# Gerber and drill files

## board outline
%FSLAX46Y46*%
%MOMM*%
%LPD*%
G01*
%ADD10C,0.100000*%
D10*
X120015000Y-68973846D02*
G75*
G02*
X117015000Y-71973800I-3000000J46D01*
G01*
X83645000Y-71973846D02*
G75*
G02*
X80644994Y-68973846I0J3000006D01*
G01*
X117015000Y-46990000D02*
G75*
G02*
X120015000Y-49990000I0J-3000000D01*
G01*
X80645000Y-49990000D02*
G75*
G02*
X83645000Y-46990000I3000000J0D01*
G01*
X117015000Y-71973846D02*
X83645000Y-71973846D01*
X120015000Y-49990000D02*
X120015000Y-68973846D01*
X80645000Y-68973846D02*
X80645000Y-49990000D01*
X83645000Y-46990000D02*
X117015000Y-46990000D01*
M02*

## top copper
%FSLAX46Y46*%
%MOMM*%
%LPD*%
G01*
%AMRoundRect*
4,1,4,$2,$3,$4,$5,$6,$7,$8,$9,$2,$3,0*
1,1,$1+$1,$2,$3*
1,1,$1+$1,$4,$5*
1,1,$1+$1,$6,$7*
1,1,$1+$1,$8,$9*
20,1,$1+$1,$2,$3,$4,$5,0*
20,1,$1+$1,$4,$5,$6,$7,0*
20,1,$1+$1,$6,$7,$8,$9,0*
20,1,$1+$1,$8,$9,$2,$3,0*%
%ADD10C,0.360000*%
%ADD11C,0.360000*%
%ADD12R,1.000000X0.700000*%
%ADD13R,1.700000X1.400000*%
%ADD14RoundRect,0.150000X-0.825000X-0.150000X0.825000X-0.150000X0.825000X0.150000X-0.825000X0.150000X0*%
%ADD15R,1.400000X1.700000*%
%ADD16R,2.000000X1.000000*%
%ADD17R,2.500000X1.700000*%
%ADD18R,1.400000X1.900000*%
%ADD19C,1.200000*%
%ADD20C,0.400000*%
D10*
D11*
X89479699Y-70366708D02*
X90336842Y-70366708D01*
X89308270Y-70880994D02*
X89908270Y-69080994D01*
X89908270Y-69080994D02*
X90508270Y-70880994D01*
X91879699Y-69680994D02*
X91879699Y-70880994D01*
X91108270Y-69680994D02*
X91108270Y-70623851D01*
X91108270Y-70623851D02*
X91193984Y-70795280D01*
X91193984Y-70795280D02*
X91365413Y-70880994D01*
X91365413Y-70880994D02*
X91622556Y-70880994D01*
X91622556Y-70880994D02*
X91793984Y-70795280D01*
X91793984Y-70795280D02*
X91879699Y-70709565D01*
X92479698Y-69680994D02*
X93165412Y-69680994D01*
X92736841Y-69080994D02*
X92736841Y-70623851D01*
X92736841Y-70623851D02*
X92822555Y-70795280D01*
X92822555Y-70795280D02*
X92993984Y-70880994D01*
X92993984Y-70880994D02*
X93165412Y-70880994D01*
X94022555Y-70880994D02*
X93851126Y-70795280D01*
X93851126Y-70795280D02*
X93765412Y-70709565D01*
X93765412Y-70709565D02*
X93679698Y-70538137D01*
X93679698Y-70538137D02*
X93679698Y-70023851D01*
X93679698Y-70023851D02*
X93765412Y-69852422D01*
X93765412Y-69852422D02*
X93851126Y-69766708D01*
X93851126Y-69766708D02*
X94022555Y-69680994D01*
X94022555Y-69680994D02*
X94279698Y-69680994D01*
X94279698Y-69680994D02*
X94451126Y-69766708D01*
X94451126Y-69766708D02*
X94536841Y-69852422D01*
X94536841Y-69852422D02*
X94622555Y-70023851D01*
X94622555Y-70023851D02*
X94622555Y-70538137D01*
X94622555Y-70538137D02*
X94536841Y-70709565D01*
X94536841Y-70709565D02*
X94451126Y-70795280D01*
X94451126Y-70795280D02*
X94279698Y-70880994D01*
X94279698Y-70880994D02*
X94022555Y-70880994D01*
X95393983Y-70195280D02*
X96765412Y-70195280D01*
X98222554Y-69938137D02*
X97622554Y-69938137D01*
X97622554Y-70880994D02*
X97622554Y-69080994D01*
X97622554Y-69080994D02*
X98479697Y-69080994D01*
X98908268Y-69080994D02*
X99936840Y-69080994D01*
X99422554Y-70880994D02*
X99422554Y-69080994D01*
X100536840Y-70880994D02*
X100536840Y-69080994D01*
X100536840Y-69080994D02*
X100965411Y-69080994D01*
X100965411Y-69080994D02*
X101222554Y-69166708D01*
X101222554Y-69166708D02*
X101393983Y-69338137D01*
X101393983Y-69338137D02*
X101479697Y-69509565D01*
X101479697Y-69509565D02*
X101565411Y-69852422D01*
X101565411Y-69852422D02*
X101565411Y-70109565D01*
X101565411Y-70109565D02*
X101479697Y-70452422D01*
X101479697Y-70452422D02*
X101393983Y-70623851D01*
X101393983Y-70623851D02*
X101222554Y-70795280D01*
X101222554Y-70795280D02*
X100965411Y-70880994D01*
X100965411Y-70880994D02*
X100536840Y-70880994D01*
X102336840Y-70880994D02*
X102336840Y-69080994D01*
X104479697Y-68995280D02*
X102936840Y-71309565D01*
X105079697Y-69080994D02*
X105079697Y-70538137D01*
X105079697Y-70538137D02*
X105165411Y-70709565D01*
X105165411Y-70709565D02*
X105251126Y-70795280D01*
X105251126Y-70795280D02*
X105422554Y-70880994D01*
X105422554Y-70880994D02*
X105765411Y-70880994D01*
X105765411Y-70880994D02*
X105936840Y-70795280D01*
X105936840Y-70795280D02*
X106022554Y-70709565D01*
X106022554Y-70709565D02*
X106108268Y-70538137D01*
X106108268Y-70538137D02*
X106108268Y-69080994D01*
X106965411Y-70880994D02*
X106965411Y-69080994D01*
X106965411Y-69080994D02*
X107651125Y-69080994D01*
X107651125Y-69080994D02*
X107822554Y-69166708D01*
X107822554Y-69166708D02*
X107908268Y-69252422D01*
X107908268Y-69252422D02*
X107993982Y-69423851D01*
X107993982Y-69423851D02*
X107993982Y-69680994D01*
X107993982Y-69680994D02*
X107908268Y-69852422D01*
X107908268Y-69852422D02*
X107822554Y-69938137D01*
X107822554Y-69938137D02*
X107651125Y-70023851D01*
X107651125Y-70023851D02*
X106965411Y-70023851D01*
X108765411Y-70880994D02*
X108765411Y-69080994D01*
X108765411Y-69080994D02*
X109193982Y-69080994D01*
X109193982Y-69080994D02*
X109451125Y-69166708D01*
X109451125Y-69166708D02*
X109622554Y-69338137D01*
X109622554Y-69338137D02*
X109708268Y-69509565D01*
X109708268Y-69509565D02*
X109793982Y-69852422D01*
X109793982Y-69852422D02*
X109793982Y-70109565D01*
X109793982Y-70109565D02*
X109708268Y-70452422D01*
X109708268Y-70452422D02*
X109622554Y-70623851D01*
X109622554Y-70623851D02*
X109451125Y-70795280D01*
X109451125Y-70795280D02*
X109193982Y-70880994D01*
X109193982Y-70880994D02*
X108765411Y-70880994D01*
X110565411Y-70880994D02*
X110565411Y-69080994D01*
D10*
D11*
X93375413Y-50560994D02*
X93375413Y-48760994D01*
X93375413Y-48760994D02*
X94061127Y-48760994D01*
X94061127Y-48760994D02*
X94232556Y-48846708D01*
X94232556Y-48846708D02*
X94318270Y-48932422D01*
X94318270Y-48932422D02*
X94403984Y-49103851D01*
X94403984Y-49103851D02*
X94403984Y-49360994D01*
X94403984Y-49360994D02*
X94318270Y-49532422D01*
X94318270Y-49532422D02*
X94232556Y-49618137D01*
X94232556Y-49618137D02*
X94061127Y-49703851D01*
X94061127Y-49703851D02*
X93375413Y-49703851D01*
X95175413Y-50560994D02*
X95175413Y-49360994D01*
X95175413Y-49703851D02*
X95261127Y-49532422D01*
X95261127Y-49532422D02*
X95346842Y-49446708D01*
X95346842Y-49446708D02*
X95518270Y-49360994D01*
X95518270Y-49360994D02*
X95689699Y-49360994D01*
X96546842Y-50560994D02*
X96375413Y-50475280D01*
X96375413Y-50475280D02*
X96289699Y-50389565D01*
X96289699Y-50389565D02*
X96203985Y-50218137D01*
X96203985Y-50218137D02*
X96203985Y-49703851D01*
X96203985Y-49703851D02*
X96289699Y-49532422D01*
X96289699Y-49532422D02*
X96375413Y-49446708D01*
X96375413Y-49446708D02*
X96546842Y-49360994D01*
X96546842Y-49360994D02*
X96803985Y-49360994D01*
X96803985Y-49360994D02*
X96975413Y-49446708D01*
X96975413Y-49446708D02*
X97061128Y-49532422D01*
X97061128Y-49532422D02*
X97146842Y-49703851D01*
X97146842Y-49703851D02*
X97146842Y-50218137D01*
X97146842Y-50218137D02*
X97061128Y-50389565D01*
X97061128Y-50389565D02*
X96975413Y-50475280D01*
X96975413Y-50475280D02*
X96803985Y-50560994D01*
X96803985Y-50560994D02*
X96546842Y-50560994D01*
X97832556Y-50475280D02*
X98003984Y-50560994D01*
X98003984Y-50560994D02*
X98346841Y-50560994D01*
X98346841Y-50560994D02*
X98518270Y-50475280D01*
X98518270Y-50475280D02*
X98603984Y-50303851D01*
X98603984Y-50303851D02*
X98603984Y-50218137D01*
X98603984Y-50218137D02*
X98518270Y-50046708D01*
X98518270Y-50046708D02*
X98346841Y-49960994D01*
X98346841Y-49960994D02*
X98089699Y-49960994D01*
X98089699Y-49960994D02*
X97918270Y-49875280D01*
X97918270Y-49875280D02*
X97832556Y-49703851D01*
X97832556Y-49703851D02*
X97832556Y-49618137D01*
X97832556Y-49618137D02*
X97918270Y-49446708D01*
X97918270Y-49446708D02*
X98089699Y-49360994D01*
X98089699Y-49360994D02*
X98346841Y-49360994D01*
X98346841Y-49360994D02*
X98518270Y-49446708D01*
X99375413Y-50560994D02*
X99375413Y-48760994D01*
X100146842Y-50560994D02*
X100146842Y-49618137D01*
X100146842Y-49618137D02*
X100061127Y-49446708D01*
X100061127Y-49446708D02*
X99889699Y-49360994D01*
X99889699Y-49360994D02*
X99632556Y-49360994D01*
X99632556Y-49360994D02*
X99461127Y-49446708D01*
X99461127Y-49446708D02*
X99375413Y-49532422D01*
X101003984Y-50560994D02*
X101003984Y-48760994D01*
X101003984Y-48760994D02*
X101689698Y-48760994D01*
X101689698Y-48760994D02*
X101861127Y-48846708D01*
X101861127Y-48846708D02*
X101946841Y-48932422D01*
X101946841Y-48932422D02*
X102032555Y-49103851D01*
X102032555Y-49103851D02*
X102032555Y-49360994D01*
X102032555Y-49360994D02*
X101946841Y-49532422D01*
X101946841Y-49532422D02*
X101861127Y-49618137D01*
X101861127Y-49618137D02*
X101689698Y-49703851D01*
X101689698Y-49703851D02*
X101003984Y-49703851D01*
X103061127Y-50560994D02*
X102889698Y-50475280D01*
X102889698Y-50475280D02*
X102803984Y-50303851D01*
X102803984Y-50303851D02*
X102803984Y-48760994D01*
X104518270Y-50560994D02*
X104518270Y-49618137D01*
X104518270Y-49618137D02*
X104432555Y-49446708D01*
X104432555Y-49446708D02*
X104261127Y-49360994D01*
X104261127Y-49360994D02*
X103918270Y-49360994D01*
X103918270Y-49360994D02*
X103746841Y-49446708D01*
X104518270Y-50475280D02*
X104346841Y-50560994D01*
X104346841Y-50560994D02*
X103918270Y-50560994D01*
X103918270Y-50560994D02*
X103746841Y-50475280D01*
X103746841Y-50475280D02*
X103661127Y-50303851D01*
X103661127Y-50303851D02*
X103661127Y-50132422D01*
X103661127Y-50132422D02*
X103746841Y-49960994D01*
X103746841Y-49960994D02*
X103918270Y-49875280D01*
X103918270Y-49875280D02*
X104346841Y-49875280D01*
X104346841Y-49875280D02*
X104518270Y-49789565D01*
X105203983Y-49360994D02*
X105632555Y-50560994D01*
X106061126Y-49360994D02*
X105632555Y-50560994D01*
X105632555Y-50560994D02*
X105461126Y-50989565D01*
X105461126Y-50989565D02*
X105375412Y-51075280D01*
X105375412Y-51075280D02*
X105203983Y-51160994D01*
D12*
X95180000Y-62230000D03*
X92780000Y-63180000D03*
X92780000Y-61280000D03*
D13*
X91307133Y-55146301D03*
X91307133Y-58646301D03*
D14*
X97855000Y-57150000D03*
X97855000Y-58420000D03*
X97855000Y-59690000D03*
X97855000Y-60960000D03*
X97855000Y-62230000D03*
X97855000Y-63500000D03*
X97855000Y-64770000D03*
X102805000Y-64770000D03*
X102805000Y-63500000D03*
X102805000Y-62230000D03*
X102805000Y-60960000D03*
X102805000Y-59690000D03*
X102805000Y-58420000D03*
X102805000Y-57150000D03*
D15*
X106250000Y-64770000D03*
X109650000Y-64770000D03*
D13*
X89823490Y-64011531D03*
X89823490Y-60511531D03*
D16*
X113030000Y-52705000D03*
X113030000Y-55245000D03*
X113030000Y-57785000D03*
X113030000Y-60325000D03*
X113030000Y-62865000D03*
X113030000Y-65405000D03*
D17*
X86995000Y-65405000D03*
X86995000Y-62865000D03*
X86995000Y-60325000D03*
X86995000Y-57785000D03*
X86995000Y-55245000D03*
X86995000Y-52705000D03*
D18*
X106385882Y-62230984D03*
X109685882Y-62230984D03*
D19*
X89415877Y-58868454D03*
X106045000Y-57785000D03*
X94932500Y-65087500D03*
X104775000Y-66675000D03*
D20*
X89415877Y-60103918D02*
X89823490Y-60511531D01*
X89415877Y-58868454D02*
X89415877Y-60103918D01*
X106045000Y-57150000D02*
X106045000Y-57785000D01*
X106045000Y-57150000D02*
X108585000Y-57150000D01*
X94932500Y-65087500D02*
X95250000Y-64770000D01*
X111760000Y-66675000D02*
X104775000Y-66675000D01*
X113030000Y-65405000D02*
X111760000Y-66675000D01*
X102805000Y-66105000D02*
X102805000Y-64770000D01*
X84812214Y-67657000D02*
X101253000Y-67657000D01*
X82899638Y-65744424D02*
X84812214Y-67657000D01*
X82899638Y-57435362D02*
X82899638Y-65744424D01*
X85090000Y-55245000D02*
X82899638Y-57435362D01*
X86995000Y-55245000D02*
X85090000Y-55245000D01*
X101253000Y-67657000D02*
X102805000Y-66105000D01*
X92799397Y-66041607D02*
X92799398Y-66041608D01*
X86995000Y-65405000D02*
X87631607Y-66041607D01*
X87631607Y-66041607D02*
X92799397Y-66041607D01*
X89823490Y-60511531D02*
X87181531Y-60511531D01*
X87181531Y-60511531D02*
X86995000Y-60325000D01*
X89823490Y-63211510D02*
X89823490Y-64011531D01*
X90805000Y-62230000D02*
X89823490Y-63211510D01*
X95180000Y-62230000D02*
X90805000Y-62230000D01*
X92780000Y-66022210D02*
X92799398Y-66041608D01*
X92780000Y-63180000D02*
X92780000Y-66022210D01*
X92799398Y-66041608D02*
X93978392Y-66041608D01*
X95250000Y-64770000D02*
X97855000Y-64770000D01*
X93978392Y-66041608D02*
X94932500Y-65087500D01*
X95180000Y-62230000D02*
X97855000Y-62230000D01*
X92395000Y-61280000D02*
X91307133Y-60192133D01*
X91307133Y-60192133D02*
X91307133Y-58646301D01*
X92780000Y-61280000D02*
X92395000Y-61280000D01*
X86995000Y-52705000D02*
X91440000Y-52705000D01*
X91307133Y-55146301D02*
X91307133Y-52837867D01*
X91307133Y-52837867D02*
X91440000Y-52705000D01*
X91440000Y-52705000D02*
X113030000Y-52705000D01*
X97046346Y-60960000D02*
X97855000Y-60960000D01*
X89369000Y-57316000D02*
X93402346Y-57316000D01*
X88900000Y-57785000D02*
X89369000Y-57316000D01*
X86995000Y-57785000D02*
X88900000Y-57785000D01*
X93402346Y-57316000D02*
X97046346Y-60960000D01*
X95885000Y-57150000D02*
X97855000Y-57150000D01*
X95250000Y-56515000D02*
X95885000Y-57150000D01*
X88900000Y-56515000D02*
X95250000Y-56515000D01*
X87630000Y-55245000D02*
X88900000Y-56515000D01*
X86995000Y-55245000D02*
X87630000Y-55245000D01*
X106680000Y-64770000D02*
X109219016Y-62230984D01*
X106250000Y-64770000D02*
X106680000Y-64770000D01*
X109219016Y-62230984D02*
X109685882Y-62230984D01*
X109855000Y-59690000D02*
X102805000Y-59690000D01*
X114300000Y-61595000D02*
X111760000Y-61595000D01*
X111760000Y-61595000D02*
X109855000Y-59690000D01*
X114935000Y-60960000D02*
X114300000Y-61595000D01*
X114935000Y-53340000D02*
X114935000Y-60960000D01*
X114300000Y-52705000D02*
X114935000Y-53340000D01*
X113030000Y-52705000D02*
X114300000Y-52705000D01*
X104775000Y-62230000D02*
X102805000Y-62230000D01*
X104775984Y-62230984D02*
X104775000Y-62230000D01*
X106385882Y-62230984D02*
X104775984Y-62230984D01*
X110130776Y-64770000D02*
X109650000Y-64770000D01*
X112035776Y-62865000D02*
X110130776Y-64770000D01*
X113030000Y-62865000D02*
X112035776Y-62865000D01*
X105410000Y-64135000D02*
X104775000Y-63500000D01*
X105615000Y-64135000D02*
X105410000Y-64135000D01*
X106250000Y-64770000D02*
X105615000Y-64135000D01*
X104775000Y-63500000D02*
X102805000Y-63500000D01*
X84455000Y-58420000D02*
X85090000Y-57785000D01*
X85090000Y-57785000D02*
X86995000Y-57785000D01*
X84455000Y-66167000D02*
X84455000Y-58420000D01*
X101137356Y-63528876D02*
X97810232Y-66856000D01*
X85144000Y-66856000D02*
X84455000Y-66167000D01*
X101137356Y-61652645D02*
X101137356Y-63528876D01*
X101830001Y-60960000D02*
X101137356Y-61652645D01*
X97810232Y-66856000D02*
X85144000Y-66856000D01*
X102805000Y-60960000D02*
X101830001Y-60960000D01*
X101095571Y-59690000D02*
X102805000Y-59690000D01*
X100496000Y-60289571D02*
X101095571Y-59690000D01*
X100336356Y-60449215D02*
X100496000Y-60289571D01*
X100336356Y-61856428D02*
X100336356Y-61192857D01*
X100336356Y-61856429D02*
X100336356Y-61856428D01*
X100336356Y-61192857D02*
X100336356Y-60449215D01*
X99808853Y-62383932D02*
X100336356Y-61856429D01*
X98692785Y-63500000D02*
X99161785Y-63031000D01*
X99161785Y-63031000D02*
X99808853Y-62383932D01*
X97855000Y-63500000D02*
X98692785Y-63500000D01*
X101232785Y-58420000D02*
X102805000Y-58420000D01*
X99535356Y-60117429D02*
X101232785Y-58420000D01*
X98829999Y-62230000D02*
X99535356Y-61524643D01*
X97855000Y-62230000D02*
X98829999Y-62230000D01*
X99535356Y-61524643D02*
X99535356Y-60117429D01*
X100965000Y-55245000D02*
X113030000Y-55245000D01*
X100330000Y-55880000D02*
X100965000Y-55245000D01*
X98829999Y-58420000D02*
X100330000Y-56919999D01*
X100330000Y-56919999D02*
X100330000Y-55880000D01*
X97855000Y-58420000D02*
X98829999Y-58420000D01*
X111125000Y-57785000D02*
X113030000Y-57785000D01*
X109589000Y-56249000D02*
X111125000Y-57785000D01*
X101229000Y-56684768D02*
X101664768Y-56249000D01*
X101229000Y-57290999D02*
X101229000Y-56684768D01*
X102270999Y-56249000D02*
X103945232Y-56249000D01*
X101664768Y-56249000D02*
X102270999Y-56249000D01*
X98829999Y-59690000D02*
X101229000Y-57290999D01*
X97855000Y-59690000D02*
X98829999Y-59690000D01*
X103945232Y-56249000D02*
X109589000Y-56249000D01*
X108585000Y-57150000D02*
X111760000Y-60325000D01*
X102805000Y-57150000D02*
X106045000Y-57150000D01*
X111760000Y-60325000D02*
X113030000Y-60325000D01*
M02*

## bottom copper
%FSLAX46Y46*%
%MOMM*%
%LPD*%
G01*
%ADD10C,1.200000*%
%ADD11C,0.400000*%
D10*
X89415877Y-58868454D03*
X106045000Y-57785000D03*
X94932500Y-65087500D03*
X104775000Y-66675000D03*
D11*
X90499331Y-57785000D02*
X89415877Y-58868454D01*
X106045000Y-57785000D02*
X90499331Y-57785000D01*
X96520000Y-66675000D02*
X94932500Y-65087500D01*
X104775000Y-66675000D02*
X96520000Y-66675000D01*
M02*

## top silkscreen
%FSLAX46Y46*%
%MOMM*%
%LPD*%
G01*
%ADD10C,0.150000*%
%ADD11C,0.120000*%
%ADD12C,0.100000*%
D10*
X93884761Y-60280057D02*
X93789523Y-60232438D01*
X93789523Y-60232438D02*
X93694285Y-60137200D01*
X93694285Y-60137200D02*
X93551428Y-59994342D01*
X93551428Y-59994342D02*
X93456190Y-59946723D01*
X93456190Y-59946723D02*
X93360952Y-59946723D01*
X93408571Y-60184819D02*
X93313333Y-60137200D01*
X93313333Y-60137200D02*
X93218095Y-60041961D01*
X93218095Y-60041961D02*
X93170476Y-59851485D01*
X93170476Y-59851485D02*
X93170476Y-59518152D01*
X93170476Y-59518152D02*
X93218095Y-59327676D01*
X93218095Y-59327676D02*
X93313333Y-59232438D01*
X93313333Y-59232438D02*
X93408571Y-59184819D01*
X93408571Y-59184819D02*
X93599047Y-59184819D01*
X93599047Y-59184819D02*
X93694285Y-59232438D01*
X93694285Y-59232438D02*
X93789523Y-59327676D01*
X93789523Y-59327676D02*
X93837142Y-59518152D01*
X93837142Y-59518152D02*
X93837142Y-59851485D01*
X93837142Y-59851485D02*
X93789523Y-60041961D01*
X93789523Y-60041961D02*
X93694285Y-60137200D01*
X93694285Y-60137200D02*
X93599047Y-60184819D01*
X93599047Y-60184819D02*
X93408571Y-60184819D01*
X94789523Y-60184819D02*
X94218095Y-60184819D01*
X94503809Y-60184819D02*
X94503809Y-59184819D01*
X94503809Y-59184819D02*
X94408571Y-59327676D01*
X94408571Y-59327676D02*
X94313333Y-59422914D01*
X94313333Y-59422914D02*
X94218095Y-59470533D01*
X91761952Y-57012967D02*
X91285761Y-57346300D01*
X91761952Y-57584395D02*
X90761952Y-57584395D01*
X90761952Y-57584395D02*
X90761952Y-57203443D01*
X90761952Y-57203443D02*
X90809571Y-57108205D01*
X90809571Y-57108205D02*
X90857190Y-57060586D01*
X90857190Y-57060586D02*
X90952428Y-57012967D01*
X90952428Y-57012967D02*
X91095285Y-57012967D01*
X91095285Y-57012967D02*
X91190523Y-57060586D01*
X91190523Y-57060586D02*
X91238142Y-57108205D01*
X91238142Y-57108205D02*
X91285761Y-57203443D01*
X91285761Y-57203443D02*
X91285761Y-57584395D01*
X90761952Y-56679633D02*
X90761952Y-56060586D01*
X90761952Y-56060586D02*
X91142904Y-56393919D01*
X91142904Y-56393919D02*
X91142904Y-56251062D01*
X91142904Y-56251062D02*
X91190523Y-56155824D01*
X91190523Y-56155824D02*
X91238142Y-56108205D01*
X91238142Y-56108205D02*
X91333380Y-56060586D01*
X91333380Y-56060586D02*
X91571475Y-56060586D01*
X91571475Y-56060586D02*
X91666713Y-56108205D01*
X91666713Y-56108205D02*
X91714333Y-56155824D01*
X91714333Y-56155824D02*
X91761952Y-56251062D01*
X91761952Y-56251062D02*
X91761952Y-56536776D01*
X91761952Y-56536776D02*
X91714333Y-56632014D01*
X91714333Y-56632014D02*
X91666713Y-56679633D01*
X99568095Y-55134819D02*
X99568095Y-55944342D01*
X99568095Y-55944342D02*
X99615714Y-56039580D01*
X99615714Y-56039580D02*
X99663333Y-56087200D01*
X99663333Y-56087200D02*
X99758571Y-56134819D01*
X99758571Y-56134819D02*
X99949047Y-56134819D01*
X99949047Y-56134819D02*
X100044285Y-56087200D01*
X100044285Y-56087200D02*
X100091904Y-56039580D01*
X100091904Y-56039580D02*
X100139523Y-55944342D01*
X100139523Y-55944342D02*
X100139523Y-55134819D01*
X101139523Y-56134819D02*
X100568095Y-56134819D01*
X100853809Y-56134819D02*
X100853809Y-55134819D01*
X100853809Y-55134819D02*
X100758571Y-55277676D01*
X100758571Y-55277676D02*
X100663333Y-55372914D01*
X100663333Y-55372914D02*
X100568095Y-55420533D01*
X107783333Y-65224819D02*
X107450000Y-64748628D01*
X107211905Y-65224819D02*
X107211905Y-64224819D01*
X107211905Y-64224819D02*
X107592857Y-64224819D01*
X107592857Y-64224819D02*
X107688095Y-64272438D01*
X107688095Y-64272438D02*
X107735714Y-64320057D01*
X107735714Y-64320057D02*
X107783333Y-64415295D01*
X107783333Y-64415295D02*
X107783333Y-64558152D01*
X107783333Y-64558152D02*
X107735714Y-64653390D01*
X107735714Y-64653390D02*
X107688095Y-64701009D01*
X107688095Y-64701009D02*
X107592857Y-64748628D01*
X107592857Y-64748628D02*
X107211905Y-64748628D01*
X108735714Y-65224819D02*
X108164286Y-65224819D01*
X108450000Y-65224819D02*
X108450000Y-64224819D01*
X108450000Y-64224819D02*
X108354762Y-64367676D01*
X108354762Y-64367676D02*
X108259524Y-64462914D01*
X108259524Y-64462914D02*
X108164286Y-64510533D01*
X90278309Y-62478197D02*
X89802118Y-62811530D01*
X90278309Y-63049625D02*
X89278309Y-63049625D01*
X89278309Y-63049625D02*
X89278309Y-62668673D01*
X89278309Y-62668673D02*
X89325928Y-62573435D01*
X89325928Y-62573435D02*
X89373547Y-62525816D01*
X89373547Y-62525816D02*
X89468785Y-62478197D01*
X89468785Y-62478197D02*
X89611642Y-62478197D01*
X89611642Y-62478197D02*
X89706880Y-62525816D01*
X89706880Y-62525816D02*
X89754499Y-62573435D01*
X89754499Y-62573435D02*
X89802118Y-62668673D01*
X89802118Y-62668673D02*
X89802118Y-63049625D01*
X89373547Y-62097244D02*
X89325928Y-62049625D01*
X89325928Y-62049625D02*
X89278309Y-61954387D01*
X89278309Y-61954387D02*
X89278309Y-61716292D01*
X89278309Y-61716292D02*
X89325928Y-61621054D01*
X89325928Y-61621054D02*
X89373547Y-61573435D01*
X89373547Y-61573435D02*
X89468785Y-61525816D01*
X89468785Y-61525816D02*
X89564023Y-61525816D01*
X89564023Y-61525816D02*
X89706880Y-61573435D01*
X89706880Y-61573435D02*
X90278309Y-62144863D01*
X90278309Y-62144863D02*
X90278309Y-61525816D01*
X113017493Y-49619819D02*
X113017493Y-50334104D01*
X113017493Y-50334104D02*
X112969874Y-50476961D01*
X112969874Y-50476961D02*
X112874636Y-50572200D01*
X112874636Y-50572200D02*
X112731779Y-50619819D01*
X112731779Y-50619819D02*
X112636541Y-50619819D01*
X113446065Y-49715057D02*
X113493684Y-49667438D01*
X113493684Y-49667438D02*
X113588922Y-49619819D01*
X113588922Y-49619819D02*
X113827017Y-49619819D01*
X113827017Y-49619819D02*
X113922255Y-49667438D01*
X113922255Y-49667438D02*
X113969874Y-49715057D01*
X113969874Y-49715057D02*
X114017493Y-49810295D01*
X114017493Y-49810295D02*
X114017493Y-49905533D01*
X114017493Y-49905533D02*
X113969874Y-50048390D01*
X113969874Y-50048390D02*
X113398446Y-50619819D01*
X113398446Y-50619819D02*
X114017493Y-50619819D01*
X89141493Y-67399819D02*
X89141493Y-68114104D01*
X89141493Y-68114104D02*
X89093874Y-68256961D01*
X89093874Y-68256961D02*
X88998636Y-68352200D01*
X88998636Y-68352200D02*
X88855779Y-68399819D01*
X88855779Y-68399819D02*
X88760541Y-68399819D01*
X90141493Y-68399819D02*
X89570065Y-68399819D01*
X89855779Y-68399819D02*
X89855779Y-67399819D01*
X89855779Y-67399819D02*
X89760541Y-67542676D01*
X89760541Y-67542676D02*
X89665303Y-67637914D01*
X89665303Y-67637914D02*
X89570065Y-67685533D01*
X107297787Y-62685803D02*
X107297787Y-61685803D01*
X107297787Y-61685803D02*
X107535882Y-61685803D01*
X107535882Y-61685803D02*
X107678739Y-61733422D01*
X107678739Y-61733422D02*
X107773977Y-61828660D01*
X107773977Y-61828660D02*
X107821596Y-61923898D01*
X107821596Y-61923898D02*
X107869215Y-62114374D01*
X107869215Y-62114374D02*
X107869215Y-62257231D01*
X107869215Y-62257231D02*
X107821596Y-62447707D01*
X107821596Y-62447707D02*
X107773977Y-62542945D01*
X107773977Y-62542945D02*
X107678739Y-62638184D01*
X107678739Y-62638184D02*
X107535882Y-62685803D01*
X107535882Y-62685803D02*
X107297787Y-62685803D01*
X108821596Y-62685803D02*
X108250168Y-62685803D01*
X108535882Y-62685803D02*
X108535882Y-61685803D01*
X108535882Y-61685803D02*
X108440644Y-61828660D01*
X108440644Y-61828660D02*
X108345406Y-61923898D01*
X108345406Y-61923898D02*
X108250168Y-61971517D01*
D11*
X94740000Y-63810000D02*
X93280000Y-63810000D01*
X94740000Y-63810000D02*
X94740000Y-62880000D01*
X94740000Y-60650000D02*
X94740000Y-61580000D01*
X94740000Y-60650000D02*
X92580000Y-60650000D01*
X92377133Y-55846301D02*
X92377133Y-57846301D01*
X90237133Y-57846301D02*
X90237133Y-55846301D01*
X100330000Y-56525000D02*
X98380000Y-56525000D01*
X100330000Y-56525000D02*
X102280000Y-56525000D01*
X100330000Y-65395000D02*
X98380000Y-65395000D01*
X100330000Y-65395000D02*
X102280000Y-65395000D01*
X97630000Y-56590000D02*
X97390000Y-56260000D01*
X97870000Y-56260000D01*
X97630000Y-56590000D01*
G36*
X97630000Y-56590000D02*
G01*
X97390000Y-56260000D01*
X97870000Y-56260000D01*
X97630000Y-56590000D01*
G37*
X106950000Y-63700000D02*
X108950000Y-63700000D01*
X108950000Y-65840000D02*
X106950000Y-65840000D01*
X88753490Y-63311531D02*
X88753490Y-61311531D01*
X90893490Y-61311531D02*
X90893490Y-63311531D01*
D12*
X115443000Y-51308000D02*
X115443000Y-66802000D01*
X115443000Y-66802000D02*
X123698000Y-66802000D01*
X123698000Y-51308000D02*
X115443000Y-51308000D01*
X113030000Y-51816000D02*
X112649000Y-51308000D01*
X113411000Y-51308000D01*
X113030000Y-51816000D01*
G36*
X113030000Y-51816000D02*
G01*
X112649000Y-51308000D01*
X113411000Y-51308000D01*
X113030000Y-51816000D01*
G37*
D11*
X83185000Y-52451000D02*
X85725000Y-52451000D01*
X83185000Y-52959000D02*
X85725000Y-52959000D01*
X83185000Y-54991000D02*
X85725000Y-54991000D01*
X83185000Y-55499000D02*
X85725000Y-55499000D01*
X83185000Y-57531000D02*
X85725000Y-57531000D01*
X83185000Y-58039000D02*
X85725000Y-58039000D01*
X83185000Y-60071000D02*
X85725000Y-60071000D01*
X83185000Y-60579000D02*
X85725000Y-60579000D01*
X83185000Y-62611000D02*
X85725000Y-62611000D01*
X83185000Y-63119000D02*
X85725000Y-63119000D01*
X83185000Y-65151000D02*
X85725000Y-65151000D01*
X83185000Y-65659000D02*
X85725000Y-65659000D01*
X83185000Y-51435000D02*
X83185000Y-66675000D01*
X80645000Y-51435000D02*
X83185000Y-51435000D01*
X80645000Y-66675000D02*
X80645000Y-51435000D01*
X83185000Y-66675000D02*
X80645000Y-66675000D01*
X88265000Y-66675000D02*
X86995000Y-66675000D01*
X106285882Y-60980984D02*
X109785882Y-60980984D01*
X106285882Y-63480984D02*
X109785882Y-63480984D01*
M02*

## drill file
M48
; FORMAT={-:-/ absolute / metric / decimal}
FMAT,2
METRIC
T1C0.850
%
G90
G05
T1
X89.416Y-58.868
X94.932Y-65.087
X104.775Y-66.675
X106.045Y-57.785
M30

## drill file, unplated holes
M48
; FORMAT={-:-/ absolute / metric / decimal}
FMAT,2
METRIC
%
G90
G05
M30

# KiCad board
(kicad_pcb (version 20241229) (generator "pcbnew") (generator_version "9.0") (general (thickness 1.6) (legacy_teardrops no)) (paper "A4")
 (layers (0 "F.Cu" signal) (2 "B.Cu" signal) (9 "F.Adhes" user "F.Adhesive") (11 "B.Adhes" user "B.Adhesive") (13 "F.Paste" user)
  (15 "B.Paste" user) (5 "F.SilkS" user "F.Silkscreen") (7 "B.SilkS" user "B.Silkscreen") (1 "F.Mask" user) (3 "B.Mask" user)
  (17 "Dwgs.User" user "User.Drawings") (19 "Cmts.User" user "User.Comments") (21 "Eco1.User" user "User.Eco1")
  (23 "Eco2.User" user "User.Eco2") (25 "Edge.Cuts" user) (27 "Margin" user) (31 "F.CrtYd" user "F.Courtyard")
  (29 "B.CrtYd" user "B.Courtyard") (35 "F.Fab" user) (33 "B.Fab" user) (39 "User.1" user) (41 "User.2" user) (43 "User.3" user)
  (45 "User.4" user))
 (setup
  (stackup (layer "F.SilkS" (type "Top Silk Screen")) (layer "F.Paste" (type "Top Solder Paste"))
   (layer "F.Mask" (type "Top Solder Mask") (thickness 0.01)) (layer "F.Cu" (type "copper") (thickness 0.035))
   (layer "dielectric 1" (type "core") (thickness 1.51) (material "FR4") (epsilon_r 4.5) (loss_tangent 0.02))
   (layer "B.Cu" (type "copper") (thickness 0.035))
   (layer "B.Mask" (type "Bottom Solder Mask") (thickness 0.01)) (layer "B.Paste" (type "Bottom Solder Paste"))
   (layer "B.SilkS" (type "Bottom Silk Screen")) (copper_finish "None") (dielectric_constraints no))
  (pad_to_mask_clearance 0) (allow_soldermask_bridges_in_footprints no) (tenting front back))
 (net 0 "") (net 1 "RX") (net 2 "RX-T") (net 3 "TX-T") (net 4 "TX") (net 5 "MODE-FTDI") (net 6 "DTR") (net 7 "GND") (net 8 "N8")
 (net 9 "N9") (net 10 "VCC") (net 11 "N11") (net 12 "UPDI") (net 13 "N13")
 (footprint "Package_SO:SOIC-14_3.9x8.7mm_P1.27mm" (layer "F.Cu") (at 100.33 60.96)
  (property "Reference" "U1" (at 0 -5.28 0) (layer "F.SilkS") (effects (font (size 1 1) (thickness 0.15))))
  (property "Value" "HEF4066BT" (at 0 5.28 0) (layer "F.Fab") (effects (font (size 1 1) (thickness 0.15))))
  (fp_line (start 0 -4.435) (end -1.95 -4.435) (stroke (width 0.12) (type solid)) (layer "F.SilkS"))
  (fp_line (start 0 -4.435) (end 1.95 -4.435) (stroke (width 0.12) (type solid)) (layer "F.SilkS"))
  (fp_line (start 0 4.435) (end -1.95 4.435) (stroke (width 0.12) (type solid)) (layer "F.SilkS"))
  (fp_line (start 0 4.435) (end 1.95 4.435) (stroke (width 0.12) (type solid)) (layer "F.SilkS"))
  (fp_poly
   (pts (xy -2.7 -4.37) (xy -2.94 -4.7) (xy -2.46 -4.7) (xy -2.7 -4.37)) (stroke (width 0.12) (type solid)) (fill yes) (layer "F.SilkS"))
  (pad "1" smd roundrect (at -2.475 -3.81) (size 1.95 0.6) (layers "F.Cu" "F.Mask" "F.Paste") (roundrect_rratio 0.25) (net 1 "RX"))
  (pad "2" smd roundrect (at -2.475 -2.54) (size 1.95 0.6) (layers "F.Cu" "F.Mask" "F.Paste") (roundrect_rratio 0.25) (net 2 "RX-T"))
  (pad "3" smd roundrect (at -2.475 -1.27) (size 1.95 0.6) (layers "F.Cu" "F.Mask" "F.Paste") (roundrect_rratio 0.25) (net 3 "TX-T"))
  (pad "4" smd roundrect (at -2.475 0) (size 1.95 0.6) (layers "F.Cu" "F.Mask" "F.Paste") (roundrect_rratio 0.25) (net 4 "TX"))
  (pad "5" smd roundrect (at -2.475 1.27) (size 1.95 0.6) (layers "F.Cu" "F.Mask" "F.Paste") (roundrect_rratio 0.25) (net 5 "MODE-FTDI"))
  (pad "6" smd roundrect (at -2.475 2.54) (size 1.95 0.6) (layers "F.Cu" "F.Mask" "F.Paste") (roundrect_rratio 0.25) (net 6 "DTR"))
  (pad "7" smd roundrect (at -2.475 3.81) (size 1.95 0.6) (layers "F.Cu" "F.Mask" "F.Paste") (roundrect_rratio 0.25) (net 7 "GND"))
  (pad "8" smd roundrect (at 2.475 3.81) (size 1.95 0.6) (layers "F.Cu" "F.Mask" "F.Paste") (roundrect_rratio 0.25) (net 1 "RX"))
  (pad "9" smd roundrect (at 2.475 2.54) (size 1.95 0.6) (layers "F.Cu" "F.Mask" "F.Paste") (roundrect_rratio 0.25) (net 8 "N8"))
  (pad "10" smd roundrect (at 2.475 1.27) (size 1.95 0.6) (layers "F.Cu" "F.Mask" "F.Paste") (roundrect_rratio 0.25) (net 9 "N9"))
  (pad "11" smd roundrect (at 2.475 0) (size 1.95 0.6) (layers "F.Cu" "F.Mask" "F.Paste") (roundrect_rratio 0.25) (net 4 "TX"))
  (pad "12" smd roundrect (at 2.475 -1.27) (size 1.95 0.6) (layers "F.Cu" "F.Mask" "F.Paste") (roundrect_rratio 0.25) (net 6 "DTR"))
  (pad "13" smd roundrect (at 2.475 -2.54) (size 1.95 0.6) (layers "F.Cu" "F.Mask" "F.Paste") (roundrect_rratio 0.25) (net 5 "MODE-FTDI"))
  (pad "14" smd roundrect (at 2.475 -3.81) (size 1.95 0.6) (layers "F.Cu" "F.Mask" "F.Paste") (roundrect_rratio 0.25) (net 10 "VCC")))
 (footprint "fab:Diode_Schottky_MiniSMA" (layer "F.Cu") (at 108.035882 62.230984)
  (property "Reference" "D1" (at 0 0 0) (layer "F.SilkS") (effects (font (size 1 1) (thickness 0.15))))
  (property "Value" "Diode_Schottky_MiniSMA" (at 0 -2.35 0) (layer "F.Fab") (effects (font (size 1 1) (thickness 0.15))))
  (fp_line (start -1.75 -1.25) (end 1.75 -1.25) (stroke (width 0.12) (type solid)) (layer "F.SilkS"))
  (fp_line (start -1.75 1.25) (end 1.75 1.25) (stroke (width 0.12) (type solid)) (layer "F.SilkS"))
  (pad "1" smd rect (at -1.65 0) (size 1.4 1.9) (layers "F.Cu" "F.Mask" "F.Paste") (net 9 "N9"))
  (pad "2" smd rect (at 1.65 0) (size 1.4 1.9) (layers "F.Cu" "F.Mask" "F.Paste") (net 8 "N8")))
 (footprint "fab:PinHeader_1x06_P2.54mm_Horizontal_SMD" (layer "F.Cu") (at 86.995 65.405 180)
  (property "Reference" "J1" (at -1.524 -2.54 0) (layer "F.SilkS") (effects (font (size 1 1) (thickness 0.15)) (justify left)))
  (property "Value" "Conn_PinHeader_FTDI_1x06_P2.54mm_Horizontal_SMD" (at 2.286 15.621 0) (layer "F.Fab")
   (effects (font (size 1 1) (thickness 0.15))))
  (fp_line (start 6.35 13.97) (end 3.81 13.97) (stroke (width 0.12) (type solid)) (layer "F.SilkS"))
  (fp_line (start 6.35 -1.27) (end 6.35 13.97) (stroke (width 0.12) (type solid)) (layer "F.SilkS"))
  (fp_line (start 3.81 13.97) (end 3.81 -1.27) (stroke (width 0.12) (type solid)) (layer "F.SilkS"))
  (fp_line (start 3.81 12.954) (end 1.27 12.954) (stroke (width 0.12) (type solid)) (layer "F.SilkS"))
  (fp_line (start 3.81 12.446) (end 1.27 12.446) (stroke (width 0.12) (type solid)) (layer "F.SilkS"))
  (fp_line (start 3.81 10.414) (end 1.27 10.414) (stroke (width 0.12) (type solid)) (layer "F.SilkS"))
  (fp_line (start 3.81 9.906) (end 1.27 9.906) (stroke (width 0.12) (type solid)) (layer "F.SilkS"))
  (fp_line (start 3.81 7.874) (end 1.27 7.874) (stroke (width 0.12) (type solid)) (layer "F.SilkS"))
  (fp_line (start 3.81 7.366) (end 1.27 7.366) (stroke (width 0.12) (type solid)) (layer "F.SilkS"))
  (fp_line (start 3.81 5.334) (end 1.27 5.334) (stroke (width 0.12) (type solid)) (layer "F.SilkS"))
  (fp_line (start 3.81 4.826) (end 1.27 4.826) (stroke (width 0.12) (type solid)) (layer "F.SilkS"))
  (fp_line (start 3.81 2.794) (end 1.27 2.794) (stroke (width 0.12) (type solid)) (layer "F.SilkS"))
  (fp_line (start 3.81 2.286) (end 1.27 2.286) (stroke (width 0.12) (type solid)) (layer "F.SilkS"))
  (fp_line (start 3.81 0.254) (end 1.27 0.254) (stroke (width 0.12) (type solid)) (layer "F.SilkS"))
  (fp_line (start 3.81 -0.254) (end 1.27 -0.254) (stroke (width 0.12) (type solid)) (layer "F.SilkS"))
  (fp_line (start 3.81 -1.27) (end 6.35 -1.27) (stroke (width 0.12) (type solid)) (layer "F.SilkS"))
  (fp_line (start -1.27 -1.27) (end 0 -1.27) (stroke (width 0.12) (type solid)) (layer "F.SilkS"))
  (pad "1" smd rect (at 0 0 180) (size 2.5 1.7) (layers "F.Cu" "F.Mask" "F.Paste") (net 7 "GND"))
  (pad "2" smd rect (at 0 2.54 180) (size 2.5 1.7) (layers "F.Cu" "F.Mask" "F.Paste") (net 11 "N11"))
  (pad "3" smd rect (at 0 5.08 180) (size 2.5 1.7) (layers "F.Cu" "F.Mask" "F.Paste") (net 10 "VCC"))
  (pad "4" smd rect (at 0 7.62 180) (size 2.5 1.7) (layers "F.Cu" "F.Mask" "F.Paste") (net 4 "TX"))
  (pad "5" smd rect (at 0 10.16 180) (size 2.5 1.7) (layers "F.Cu" "F.Mask" "F.Paste") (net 1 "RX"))
  (pad "6" smd rect (at 0 12.7 180) (size 2.5 1.7) (layers "F.Cu" "F.Mask" "F.Paste") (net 6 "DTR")))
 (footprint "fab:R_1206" (layer "F.Cu") (at 107.95 64.77)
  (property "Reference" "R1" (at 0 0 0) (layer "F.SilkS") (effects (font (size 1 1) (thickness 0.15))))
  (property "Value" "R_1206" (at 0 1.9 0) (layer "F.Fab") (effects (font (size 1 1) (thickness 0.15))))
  (fp_line (start -1 -1.07) (end 1 -1.07) (stroke (width 0.12) (type solid)) (layer "F.SilkS"))
  (fp_line (start 1 1.07) (end -1 1.07) (stroke (width 0.12) (type solid)) (layer "F.SilkS"))
  (pad "1" smd rect (at -1.7 0) (size 1.4 1.7) (layers "F.Cu" "F.Mask" "F.Paste") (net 8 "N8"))
  (pad "2" smd rect (at 1.7 0) (size 1.4 1.7) (layers "F.Cu" "F.Mask" "F.Paste") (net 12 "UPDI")))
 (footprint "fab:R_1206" (layer "F.Cu") (at 91.307133 56.846301 90)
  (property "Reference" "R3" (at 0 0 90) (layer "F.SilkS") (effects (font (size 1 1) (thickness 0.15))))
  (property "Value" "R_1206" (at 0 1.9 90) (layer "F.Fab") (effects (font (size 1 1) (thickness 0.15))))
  (fp_line (start -1 -1.07) (end 1 -1.07) (stroke (width 0.12) (type solid)) (layer "F.SilkS"))
  (fp_line (start 1 1.07) (end -1 1.07) (stroke (width 0.12) (type solid)) (layer "F.SilkS"))
  (pad "1" smd rect (at -1.8 0 90) (size 1.4 1.7) (layers "F.Cu" "F.Mask" "F.Paste") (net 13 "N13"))
  (pad "2" smd rect (at 1.7 0 90) (size 1.4 1.7) (layers "F.Cu" "F.Mask" "F.Paste") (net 6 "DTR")))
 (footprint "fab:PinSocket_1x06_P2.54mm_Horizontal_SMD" (layer "F.Cu") (at 113.03 52.705)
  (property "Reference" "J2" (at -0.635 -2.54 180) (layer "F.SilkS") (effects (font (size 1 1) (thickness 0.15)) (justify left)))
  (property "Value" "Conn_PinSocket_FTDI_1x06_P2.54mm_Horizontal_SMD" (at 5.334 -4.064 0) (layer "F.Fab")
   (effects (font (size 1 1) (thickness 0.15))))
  (fp_line (start 2.413 -1.397) (end 2.413 14.097) (stroke (width 0.1) (type default)) (layer "F.SilkS"))
  (fp_line (start 2.413 14.097) (end 10.668 14.097) (stroke (width 0.1) (type default)) (layer "F.SilkS"))
  (fp_line (start 10.668 -1.397) (end 2.413 -1.397) (stroke (width 0.1) (type default)) (layer "F.SilkS"))
  (fp_poly (pts (xy 0 -0.889) (xy -0.381 -1.397) (xy 0.381 -1.397)) (stroke (width 0.1) (type solid)) (fill yes) (layer "F.SilkS"))
  (pad "1" smd rect (at 0 0) (size 2 1) (layers "F.Cu" "F.Mask" "F.Paste") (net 6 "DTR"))
  (pad "2" smd rect (at 0 2.54) (size 2 1) (layers "F.Cu" "F.Mask" "F.Paste") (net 2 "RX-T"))
  (pad "3" smd rect (at 0 5.08) (size 2 1) (layers "F.Cu" "F.Mask" "F.Paste") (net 3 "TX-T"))
  (pad "4" smd rect (at 0 7.62) (size 2 1) (layers "F.Cu" "F.Mask" "F.Paste") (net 10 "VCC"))
  (pad "5" smd rect (at 0 10.16) (size 2 1) (layers "F.Cu" "F.Mask" "F.Paste") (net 12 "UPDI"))
  (pad "6" smd rect (at 0 12.7) (size 2 1) (layers "F.Cu" "F.Mask" "F.Paste") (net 7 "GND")))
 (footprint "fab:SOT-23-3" (layer "F.Cu") (at 93.98 62.23)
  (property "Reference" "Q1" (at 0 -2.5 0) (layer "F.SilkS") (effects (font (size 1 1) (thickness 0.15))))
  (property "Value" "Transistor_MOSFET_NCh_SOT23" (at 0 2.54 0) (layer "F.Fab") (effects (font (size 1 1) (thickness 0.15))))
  (fp_line (start 0.76 -1.58) (end -1.4 -1.58) (stroke (width 0.12) (type solid)) (layer "F.SilkS"))
  (fp_line (start 0.76 -1.58) (end 0.76 -0.65) (stroke (width 0.12) (type solid)) (layer "F.SilkS"))
  (fp_line (start 0.76 1.58) (end -0.7 1.58) (stroke (width 0.12) (type solid)) (layer "F.SilkS"))
  (fp_line (start 0.76 1.58) (end 0.76 0.65) (stroke (width 0.12) (type solid)) (layer "F.SilkS"))
  (pad "1" smd rect (at -1.2 -0.95) (size 1 0.7) (layers "F.Cu" "F.Mask" "F.Paste") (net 13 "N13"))
  (pad "2" smd rect (at -1.2 0.95) (size 1 0.7) (layers "F.Cu" "F.Mask" "F.Paste") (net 7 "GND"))
  (pad "3" smd rect (at 1.2 0) (size 1 0.7) (layers "F.Cu" "F.Mask" "F.Paste") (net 5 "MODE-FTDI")))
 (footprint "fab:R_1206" (layer "F.Cu") (at 89.82349 62.311531 90)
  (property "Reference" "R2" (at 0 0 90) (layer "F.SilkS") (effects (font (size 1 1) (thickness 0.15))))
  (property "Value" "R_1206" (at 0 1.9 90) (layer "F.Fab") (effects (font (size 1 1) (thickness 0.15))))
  (fp_line (start -1 -1.07) (end 1 -1.07) (stroke (width 0.12) (type solid)) (layer "F.SilkS"))
  (fp_line (start 1 1.07) (end -1 1.07) (stroke (width 0.12) (type solid)) (layer "F.SilkS"))
  (pad "1" smd rect (at -1.7 0 90) (size 1.4 1.7) (layers "F.Cu" "F.Mask" "F.Paste") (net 5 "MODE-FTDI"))
  (pad "2" smd rect (at 1.8 0 90) (size 1.4 1.7) (layers "F.Cu" "F.Mask" "F.Paste") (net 10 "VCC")))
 (gr_line (start 80.645 68.973846) (end 80.645 49.99) (stroke (width 0.1) (type default)) (layer "Edge.Cuts"))
 (gr_line (start 117.015 71.973846) (end 83.645 71.973846) (stroke (width 0.1) (type default)) (layer "Edge.Cuts"))
 (gr_arc (start 80.645 49.99) (mid 81.52368 47.86868) (end 83.645 46.99) (stroke (width 0.1) (type default)) (layer "Edge.Cuts"))
 (gr_line (start 120.015 49.99) (end 120.015 68.973846) (stroke (width 0.1) (type default)) (layer "Edge.Cuts"))
 (gr_arc (start 117.015 46.99) (mid 119.13632 47.86868) (end 120.015 49.99) (stroke (width 0.1) (type default)) (layer "Edge.Cuts"))
 (gr_line (start 83.645 46.99) (end 117.015 46.99) (stroke (width 0.1) (type default)) (layer "Edge.Cuts"))
 (gr_arc (start 120.015 68.973846) (mid 119.13632 71.095166) (end 117.015 71.973846) (stroke (width 0.1) (type default)) (layer "Edge.Cuts"))
 (gr_arc (start 83.645 71.973846) (mid 81.523678 71.095167) (end 80.645 68.973846) (stroke (width 0.1) (type default)) (layer "Edge.Cuts"))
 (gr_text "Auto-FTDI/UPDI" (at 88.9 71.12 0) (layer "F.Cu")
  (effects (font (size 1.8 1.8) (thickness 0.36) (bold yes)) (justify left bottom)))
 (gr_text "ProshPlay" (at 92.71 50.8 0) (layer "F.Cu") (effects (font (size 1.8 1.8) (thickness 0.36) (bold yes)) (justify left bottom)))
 (segment (start 106.25 64.77) (end 105.615 64.135) (width 0.4) (layer "F.Cu") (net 8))
 (segment (start 105.41 64.135) (end 104.775 63.5) (width 0.4) (layer "F.Cu") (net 8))
 (segment (start 109.219016 62.230984) (end 109.685882 62.230984) (width 0.4) (layer "F.Cu") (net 8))
 (segment (start 106.68 64.77) (end 109.219016 62.230984) (width 0.4) (layer "F.Cu") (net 8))
 (segment (start 104.775 63.5) (end 102.805 63.5) (width 0.4) (layer "F.Cu") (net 8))
 (segment (start 106.25 64.77) (end 106.68 64.77) (width 0.4) (layer "F.Cu") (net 8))
 (segment (start 105.615 64.135) (end 105.41 64.135) (width 0.4) (layer "F.Cu") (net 8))
 (segment (start 104.775984 62.230984) (end 104.775 62.23) (width 0.4) (layer "F.Cu") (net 9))
 (segment (start 104.775 62.23) (end 102.805 62.23) (width 0.4) (layer "F.Cu") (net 9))
 (segment (start 106.385882 62.230984) (end 104.775984 62.230984) (width 0.4) (layer "F.Cu") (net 9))
 (segment (start 102.805 57.15) (end 106.045 57.15) (width 0.4) (layer "F.Cu") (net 10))
 (segment (start 89.82349 60.511531) (end 87.181531 60.511531) (width 0.4) (layer "F.Cu") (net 10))
 (segment (start 111.76 60.325) (end 113.03 60.325) (width 0.4) (layer "F.Cu") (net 10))
 (segment (start 89.415877 58.868454) (end 89.415877 60.103918) (width 0.4) (layer "F.Cu") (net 10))
 (segment (start 106.045 57.15) (end 106.045 57.785) (width 0.4) (layer "F.Cu") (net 10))
 (segment (start 87.181531 60.511531) (end 86.995 60.325) (width 0.4) (layer "F.Cu") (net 10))
 (segment (start 106.045 57.15) (end 108.585 57.15) (width 0.4) (layer "F.Cu") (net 10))
 (segment (start 108.585 57.15) (end 111.76 60.325) (width 0.4) (layer "F.Cu") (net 10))
 (segment (start 89.415877 60.103918) (end 89.82349 60.511531) (width 0.4) (layer "F.Cu") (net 10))
 (via (at 106.045 57.785) (size 1.2) (drill 0.85) (layers "F.Cu" "B.Cu") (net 10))
 (via (at 89.415877 58.868454) (size 1.2) (drill 0.85) (layers "F.Cu" "B.Cu") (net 10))
 (segment (start 106.045 57.785) (end 90.499331 57.785) (width 0.4) (layer "B.Cu") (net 10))
 (segment (start 90.499331 57.785) (end 89.415877 58.868454) (width 0.4) (layer "B.Cu") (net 10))
 (segment (start 92.78 63.18) (end 92.78 66.02221) (width 0.4) (layer "F.Cu") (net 7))
 (segment (start 92.78 66.02221) (end 92.799398 66.041608) (width 0.4) (layer "F.Cu") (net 7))
 (segment (start 94.9325 65.0875) (end 95.25 64.77) (width 0.4) (layer "F.Cu") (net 7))
 (segment (start 113.03 65.405) (end 111.76 66.675) (width 0.4) (layer "F.Cu") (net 7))
 (segment (start 92.799397 66.041607) (end 92.799398 66.041608) (width 0.4) (layer "F.Cu") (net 7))
 (segment (start 92.799398 66.041608) (end 93.978392 66.041608) (width 0.4) (layer "F.Cu") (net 7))
 (segment (start 86.995 65.405) (end 87.631607 66.041607) (width 0.4) (layer "F.Cu") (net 7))
 (segment (start 93.978392 66.041608) (end 94.9325 65.0875) (width 0.4) (layer "F.Cu") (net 7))
 (segment (start 111.76 66.675) (end 104.775 66.675) (width 0.4) (layer "F.Cu") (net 7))
 (segment (start 95.25 64.77) (end 97.855 64.77) (width 0.4) (layer "F.Cu") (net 7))
 (segment (start 87.631607 66.041607) (end 92.799397 66.041607) (width 0.4) (layer "F.Cu") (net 7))
 (via (at 104.775 66.675) (size 1.2) (drill 0.85) (layers "F.Cu" "B.Cu") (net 7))
 (via (at 94.9325 65.0875) (size 1.2) (drill 0.85) (layers "F.Cu" "B.Cu") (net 7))
 (segment (start 96.52 66.675) (end 94.9325 65.0875) (width 0.4) (layer "B.Cu") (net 7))
 (segment (start 104.775 66.675) (end 96.52 66.675) (width 0.4) (layer "B.Cu") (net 7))
 (segment (start 114.3 52.705) (end 114.935 53.34) (width 0.4) (layer "F.Cu") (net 6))
 (segment (start 100.496 60.289571) (end 101.095571 59.69) (width 0.4) (layer "F.Cu") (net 6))
 (segment (start 98.692785 63.5) (end 99.161785 63.031) (width 0.4) (layer "F.Cu") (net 6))
 (segment (start 100.336356 61.192857) (end 100.336356 60.449215) (width 0.4) (layer "F.Cu") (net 6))
 (segment (start 100.336356 61.856428) (end 100.336356 61.192857) (width 0.4) (layer "F.Cu") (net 6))
 (segment (start 100.336356 60.449215) (end 100.496 60.289571) (width 0.4) (layer "F.Cu") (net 6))
 (segment (start 114.3 61.595) (end 111.76 61.595) (width 0.4) (layer "F.Cu") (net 6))
 (segment (start 86.995 52.705) (end 91.44 52.705) (width 0.4) (layer "F.Cu") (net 6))
 (segment (start 101.095571 59.69) (end 102.805 59.69) (width 0.4) (layer "F.Cu") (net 6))
 (segment (start 111.76 61.595) (end 109.855 59.69) (width 0.4) (layer "F.Cu") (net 6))
 (segment (start 91.307133 52.837867) (end 91.44 52.705) (width 0.4) (layer "F.Cu") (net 6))
 (segment (start 97.855 63.5) (end 98.692785 63.5) (width 0.4) (layer "F.Cu") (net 6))
 (segment (start 99.161785 63.031) (end 99.808853 62.383932) (width 0.4) (layer "F.Cu") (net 6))
 (segment (start 91.307133 55.146301) (end 91.307133 52.837867) (width 0.4) (layer "F.Cu") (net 6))
 (segment (start 113.03 52.705) (end 114.3 52.705) (width 0.4) (layer "F.Cu") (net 6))
 (segment (start 109.855 59.69) (end 102.805 59.69) (width 0.4) (layer "F.Cu") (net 6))
 (segment (start 99.808853 62.383932) (end 100.336356 61.856429) (width 0.4) (layer "F.Cu") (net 6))
 (segment (start 114.935 53.34) (end 114.935 60.96) (width 0.4) (layer "F.Cu") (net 6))
 (segment (start 91.44 52.705) (end 113.03 52.705) (width 0.4) (layer "F.Cu") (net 6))
 (segment (start 100.336356 61.856429) (end 100.336356 61.856428) (width 0.4) (layer "F.Cu") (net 6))
 (segment (start 114.935 60.96) (end 114.3 61.595) (width 0.4) (layer "F.Cu") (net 6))
 (segment (start 82.899638 65.744424) (end 84.812214 67.657) (width 0.4) (layer "F.Cu") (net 1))
 (segment (start 87.63 55.245) (end 88.9 56.515) (width 0.4) (layer "F.Cu") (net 1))
 (segment (start 88.9 56.515) (end 95.25 56.515) (width 0.4) (layer "F.Cu") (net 1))
 (segment (start 85.09 55.245) (end 82.899638 57.435362) (width 0.4) (layer "F.Cu") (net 1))
 (segment (start 84.812214 67.657) (end 101.253 67.657) (width 0.4) (layer "F.Cu") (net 1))
 (segment (start 101.253 67.657) (end 102.805 66.105) (width 0.4) (layer "F.Cu") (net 1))
 (segment (start 95.885 57.15) (end 97.855 57.15) (width 0.4) (layer "F.Cu") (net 1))
 (segment (start 82.899638 57.435362) (end 82.899638 65.744424) (width 0.4) (layer "F.Cu") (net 1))
 (segment (start 86.995 55.245) (end 87.63 55.245) (width 0.4) (layer "F.Cu") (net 1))
 (segment (start 95.25 56.515) (end 95.885 57.15) (width 0.4) (layer "F.Cu") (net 1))
 (segment (start 86.995 55.245) (end 85.09 55.245) (width 0.4) (layer "F.Cu") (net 1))
 (segment (start 102.805 66.105) (end 102.805 64.77) (width 0.4) (layer "F.Cu") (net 1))
 (segment (start 85.144 66.856) (end 84.455 66.167) (width 0.4) (layer "F.Cu") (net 4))
 (segment (start 101.137356 61.652645) (end 101.137356 63.528876) (width 0.4) (layer "F.Cu") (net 4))
 (segment (start 88.9 57.785) (end 89.369 57.316) (width 0.4) (layer "F.Cu") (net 4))
 (segment (start 102.805 60.96) (end 101.830001 60.96) (width 0.4) (layer "F.Cu") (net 4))
 (segment (start 97.046346 60.96) (end 97.855 60.96) (width 0.4) (layer "F.Cu") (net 4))
 (segment (start 93.402346 57.316) (end 97.046346 60.96) (width 0.4) (layer "F.Cu") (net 4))
 (segment (start 86.995 57.785) (end 88.9 57.785) (width 0.4) (layer "F.Cu") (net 4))
 (segment (start 84.455 58.42) (end 85.09 57.785) (width 0.4) (layer "F.Cu") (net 4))
 (segment (start 97.810232 66.856) (end 85.144 66.856) (width 0.4) (layer "F.Cu") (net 4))
 (segment (start 85.09 57.785) (end 86.995 57.785) (width 0.4) (layer "F.Cu") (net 4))
 (segment (start 84.455 66.167) (end 84.455 58.42) (width 0.4) (layer "F.Cu") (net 4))
 (segment (start 101.830001 60.96) (end 101.137356 61.652645) (width 0.4) (layer "F.Cu") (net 4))
 (segment (start 101.137356 63.528876) (end 97.810232 66.856) (width 0.4) (layer "F.Cu") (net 4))
 (segment (start 89.369 57.316) (end 93.402346 57.316) (width 0.4) (layer "F.Cu") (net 4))
 (segment (start 97.855 58.42) (end 98.829999 58.42) (width 0.4) (layer "F.Cu") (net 2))
 (segment (start 100.33 56.919999) (end 100.33 55.88) (width 0.4) (layer "F.Cu") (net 2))
 (segment (start 100.965 55.245) (end 113.03 55.245) (width 0.4) (layer "F.Cu") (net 2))
 (segment (start 98.829999 58.42) (end 100.33 56.919999) (width 0.4) (layer "F.Cu") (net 2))
 (segment (start 100.33 55.88) (end 100.965 55.245) (width 0.4) (layer "F.Cu") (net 2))
 (segment (start 110.130776 64.77) (end 109.65 64.77) (width 0.4) (layer "F.Cu") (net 12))
 (segment (start 113.03 62.865) (end 112.035776 62.865) (width 0.4) (layer "F.Cu") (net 12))
 (segment (start 112.035776 62.865) (end 110.130776 64.77) (width 0.4) (layer "F.Cu") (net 12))
 (segment (start 102.270999 56.249) (end 103.945232 56.249) (width 0.4) (layer "F.Cu") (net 3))
 (segment (start 101.664768 56.249) (end 102.270999 56.249) (width 0.4) (layer "F.Cu") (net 3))
 (segment (start 101.229 56.684768) (end 101.664768 56.249) (width 0.4) (layer "F.Cu") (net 3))
 (segment (start 98.829999 59.69) (end 101.229 57.290999) (width 0.4) (layer "F.Cu") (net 3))
 (segment (start 109.589 56.249) (end 111.125 57.785) (width 0.4) (layer "F.Cu") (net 3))
 (segment (start 103.945232 56.249) (end 109.589 56.249) (width 0.4) (layer "F.Cu") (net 3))
 (segment (start 111.125 57.785) (end 113.03 57.785) (width 0.4) (layer "F.Cu") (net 3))
 (segment (start 97.855 59.69) (end 98.829999 59.69) (width 0.4) (layer "F.Cu") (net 3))
 (segment (start 101.229 57.290999) (end 101.229 56.684768) (width 0.4) (layer "F.Cu") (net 3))
 (segment (start 89.82349 63.21151) (end 89.82349 64.011531) (width 0.4) (layer "F.Cu") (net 5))
 (segment (start 99.535356 60.117429) (end 101.232785 58.42) (width 0.4) (layer "F.Cu") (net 5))
 (segment (start 97.855 62.23) (end 98.829999 62.23) (width 0.4) (layer "F.Cu") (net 5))
 (segment (start 101.232785 58.42) (end 102.805 58.42) (width 0.4) (layer "F.Cu") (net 5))
 (segment (start 95.18 62.23) (end 97.855 62.23) (width 0.4) (layer "F.Cu") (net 5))
 (segment (start 98.829999 62.23) (end 99.535356 61.524643) (width 0.4) (layer "F.Cu") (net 5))
 (segment (start 90.805 62.23) (end 89.82349 63.21151) (width 0.4) (layer "F.Cu") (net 5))
 (segment (start 95.18 62.23) (end 90.805 62.23) (width 0.4) (layer "F.Cu") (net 5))
 (segment (start 99.535356 61.524643) (end 99.535356 60.117429) (width 0.4) (layer "F.Cu") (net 5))
 (segment (start 91.307133 60.192133) (end 91.307133 58.646301) (width 0.4) (layer "F.Cu") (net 13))
 (segment (start 92.395 61.28) (end 91.307133 60.192133) (width 0.4) (layer "F.Cu") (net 13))
 (segment (start 92.78 61.28) (end 92.395 61.28) (width 0.4) (layer "F.Cu") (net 13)))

